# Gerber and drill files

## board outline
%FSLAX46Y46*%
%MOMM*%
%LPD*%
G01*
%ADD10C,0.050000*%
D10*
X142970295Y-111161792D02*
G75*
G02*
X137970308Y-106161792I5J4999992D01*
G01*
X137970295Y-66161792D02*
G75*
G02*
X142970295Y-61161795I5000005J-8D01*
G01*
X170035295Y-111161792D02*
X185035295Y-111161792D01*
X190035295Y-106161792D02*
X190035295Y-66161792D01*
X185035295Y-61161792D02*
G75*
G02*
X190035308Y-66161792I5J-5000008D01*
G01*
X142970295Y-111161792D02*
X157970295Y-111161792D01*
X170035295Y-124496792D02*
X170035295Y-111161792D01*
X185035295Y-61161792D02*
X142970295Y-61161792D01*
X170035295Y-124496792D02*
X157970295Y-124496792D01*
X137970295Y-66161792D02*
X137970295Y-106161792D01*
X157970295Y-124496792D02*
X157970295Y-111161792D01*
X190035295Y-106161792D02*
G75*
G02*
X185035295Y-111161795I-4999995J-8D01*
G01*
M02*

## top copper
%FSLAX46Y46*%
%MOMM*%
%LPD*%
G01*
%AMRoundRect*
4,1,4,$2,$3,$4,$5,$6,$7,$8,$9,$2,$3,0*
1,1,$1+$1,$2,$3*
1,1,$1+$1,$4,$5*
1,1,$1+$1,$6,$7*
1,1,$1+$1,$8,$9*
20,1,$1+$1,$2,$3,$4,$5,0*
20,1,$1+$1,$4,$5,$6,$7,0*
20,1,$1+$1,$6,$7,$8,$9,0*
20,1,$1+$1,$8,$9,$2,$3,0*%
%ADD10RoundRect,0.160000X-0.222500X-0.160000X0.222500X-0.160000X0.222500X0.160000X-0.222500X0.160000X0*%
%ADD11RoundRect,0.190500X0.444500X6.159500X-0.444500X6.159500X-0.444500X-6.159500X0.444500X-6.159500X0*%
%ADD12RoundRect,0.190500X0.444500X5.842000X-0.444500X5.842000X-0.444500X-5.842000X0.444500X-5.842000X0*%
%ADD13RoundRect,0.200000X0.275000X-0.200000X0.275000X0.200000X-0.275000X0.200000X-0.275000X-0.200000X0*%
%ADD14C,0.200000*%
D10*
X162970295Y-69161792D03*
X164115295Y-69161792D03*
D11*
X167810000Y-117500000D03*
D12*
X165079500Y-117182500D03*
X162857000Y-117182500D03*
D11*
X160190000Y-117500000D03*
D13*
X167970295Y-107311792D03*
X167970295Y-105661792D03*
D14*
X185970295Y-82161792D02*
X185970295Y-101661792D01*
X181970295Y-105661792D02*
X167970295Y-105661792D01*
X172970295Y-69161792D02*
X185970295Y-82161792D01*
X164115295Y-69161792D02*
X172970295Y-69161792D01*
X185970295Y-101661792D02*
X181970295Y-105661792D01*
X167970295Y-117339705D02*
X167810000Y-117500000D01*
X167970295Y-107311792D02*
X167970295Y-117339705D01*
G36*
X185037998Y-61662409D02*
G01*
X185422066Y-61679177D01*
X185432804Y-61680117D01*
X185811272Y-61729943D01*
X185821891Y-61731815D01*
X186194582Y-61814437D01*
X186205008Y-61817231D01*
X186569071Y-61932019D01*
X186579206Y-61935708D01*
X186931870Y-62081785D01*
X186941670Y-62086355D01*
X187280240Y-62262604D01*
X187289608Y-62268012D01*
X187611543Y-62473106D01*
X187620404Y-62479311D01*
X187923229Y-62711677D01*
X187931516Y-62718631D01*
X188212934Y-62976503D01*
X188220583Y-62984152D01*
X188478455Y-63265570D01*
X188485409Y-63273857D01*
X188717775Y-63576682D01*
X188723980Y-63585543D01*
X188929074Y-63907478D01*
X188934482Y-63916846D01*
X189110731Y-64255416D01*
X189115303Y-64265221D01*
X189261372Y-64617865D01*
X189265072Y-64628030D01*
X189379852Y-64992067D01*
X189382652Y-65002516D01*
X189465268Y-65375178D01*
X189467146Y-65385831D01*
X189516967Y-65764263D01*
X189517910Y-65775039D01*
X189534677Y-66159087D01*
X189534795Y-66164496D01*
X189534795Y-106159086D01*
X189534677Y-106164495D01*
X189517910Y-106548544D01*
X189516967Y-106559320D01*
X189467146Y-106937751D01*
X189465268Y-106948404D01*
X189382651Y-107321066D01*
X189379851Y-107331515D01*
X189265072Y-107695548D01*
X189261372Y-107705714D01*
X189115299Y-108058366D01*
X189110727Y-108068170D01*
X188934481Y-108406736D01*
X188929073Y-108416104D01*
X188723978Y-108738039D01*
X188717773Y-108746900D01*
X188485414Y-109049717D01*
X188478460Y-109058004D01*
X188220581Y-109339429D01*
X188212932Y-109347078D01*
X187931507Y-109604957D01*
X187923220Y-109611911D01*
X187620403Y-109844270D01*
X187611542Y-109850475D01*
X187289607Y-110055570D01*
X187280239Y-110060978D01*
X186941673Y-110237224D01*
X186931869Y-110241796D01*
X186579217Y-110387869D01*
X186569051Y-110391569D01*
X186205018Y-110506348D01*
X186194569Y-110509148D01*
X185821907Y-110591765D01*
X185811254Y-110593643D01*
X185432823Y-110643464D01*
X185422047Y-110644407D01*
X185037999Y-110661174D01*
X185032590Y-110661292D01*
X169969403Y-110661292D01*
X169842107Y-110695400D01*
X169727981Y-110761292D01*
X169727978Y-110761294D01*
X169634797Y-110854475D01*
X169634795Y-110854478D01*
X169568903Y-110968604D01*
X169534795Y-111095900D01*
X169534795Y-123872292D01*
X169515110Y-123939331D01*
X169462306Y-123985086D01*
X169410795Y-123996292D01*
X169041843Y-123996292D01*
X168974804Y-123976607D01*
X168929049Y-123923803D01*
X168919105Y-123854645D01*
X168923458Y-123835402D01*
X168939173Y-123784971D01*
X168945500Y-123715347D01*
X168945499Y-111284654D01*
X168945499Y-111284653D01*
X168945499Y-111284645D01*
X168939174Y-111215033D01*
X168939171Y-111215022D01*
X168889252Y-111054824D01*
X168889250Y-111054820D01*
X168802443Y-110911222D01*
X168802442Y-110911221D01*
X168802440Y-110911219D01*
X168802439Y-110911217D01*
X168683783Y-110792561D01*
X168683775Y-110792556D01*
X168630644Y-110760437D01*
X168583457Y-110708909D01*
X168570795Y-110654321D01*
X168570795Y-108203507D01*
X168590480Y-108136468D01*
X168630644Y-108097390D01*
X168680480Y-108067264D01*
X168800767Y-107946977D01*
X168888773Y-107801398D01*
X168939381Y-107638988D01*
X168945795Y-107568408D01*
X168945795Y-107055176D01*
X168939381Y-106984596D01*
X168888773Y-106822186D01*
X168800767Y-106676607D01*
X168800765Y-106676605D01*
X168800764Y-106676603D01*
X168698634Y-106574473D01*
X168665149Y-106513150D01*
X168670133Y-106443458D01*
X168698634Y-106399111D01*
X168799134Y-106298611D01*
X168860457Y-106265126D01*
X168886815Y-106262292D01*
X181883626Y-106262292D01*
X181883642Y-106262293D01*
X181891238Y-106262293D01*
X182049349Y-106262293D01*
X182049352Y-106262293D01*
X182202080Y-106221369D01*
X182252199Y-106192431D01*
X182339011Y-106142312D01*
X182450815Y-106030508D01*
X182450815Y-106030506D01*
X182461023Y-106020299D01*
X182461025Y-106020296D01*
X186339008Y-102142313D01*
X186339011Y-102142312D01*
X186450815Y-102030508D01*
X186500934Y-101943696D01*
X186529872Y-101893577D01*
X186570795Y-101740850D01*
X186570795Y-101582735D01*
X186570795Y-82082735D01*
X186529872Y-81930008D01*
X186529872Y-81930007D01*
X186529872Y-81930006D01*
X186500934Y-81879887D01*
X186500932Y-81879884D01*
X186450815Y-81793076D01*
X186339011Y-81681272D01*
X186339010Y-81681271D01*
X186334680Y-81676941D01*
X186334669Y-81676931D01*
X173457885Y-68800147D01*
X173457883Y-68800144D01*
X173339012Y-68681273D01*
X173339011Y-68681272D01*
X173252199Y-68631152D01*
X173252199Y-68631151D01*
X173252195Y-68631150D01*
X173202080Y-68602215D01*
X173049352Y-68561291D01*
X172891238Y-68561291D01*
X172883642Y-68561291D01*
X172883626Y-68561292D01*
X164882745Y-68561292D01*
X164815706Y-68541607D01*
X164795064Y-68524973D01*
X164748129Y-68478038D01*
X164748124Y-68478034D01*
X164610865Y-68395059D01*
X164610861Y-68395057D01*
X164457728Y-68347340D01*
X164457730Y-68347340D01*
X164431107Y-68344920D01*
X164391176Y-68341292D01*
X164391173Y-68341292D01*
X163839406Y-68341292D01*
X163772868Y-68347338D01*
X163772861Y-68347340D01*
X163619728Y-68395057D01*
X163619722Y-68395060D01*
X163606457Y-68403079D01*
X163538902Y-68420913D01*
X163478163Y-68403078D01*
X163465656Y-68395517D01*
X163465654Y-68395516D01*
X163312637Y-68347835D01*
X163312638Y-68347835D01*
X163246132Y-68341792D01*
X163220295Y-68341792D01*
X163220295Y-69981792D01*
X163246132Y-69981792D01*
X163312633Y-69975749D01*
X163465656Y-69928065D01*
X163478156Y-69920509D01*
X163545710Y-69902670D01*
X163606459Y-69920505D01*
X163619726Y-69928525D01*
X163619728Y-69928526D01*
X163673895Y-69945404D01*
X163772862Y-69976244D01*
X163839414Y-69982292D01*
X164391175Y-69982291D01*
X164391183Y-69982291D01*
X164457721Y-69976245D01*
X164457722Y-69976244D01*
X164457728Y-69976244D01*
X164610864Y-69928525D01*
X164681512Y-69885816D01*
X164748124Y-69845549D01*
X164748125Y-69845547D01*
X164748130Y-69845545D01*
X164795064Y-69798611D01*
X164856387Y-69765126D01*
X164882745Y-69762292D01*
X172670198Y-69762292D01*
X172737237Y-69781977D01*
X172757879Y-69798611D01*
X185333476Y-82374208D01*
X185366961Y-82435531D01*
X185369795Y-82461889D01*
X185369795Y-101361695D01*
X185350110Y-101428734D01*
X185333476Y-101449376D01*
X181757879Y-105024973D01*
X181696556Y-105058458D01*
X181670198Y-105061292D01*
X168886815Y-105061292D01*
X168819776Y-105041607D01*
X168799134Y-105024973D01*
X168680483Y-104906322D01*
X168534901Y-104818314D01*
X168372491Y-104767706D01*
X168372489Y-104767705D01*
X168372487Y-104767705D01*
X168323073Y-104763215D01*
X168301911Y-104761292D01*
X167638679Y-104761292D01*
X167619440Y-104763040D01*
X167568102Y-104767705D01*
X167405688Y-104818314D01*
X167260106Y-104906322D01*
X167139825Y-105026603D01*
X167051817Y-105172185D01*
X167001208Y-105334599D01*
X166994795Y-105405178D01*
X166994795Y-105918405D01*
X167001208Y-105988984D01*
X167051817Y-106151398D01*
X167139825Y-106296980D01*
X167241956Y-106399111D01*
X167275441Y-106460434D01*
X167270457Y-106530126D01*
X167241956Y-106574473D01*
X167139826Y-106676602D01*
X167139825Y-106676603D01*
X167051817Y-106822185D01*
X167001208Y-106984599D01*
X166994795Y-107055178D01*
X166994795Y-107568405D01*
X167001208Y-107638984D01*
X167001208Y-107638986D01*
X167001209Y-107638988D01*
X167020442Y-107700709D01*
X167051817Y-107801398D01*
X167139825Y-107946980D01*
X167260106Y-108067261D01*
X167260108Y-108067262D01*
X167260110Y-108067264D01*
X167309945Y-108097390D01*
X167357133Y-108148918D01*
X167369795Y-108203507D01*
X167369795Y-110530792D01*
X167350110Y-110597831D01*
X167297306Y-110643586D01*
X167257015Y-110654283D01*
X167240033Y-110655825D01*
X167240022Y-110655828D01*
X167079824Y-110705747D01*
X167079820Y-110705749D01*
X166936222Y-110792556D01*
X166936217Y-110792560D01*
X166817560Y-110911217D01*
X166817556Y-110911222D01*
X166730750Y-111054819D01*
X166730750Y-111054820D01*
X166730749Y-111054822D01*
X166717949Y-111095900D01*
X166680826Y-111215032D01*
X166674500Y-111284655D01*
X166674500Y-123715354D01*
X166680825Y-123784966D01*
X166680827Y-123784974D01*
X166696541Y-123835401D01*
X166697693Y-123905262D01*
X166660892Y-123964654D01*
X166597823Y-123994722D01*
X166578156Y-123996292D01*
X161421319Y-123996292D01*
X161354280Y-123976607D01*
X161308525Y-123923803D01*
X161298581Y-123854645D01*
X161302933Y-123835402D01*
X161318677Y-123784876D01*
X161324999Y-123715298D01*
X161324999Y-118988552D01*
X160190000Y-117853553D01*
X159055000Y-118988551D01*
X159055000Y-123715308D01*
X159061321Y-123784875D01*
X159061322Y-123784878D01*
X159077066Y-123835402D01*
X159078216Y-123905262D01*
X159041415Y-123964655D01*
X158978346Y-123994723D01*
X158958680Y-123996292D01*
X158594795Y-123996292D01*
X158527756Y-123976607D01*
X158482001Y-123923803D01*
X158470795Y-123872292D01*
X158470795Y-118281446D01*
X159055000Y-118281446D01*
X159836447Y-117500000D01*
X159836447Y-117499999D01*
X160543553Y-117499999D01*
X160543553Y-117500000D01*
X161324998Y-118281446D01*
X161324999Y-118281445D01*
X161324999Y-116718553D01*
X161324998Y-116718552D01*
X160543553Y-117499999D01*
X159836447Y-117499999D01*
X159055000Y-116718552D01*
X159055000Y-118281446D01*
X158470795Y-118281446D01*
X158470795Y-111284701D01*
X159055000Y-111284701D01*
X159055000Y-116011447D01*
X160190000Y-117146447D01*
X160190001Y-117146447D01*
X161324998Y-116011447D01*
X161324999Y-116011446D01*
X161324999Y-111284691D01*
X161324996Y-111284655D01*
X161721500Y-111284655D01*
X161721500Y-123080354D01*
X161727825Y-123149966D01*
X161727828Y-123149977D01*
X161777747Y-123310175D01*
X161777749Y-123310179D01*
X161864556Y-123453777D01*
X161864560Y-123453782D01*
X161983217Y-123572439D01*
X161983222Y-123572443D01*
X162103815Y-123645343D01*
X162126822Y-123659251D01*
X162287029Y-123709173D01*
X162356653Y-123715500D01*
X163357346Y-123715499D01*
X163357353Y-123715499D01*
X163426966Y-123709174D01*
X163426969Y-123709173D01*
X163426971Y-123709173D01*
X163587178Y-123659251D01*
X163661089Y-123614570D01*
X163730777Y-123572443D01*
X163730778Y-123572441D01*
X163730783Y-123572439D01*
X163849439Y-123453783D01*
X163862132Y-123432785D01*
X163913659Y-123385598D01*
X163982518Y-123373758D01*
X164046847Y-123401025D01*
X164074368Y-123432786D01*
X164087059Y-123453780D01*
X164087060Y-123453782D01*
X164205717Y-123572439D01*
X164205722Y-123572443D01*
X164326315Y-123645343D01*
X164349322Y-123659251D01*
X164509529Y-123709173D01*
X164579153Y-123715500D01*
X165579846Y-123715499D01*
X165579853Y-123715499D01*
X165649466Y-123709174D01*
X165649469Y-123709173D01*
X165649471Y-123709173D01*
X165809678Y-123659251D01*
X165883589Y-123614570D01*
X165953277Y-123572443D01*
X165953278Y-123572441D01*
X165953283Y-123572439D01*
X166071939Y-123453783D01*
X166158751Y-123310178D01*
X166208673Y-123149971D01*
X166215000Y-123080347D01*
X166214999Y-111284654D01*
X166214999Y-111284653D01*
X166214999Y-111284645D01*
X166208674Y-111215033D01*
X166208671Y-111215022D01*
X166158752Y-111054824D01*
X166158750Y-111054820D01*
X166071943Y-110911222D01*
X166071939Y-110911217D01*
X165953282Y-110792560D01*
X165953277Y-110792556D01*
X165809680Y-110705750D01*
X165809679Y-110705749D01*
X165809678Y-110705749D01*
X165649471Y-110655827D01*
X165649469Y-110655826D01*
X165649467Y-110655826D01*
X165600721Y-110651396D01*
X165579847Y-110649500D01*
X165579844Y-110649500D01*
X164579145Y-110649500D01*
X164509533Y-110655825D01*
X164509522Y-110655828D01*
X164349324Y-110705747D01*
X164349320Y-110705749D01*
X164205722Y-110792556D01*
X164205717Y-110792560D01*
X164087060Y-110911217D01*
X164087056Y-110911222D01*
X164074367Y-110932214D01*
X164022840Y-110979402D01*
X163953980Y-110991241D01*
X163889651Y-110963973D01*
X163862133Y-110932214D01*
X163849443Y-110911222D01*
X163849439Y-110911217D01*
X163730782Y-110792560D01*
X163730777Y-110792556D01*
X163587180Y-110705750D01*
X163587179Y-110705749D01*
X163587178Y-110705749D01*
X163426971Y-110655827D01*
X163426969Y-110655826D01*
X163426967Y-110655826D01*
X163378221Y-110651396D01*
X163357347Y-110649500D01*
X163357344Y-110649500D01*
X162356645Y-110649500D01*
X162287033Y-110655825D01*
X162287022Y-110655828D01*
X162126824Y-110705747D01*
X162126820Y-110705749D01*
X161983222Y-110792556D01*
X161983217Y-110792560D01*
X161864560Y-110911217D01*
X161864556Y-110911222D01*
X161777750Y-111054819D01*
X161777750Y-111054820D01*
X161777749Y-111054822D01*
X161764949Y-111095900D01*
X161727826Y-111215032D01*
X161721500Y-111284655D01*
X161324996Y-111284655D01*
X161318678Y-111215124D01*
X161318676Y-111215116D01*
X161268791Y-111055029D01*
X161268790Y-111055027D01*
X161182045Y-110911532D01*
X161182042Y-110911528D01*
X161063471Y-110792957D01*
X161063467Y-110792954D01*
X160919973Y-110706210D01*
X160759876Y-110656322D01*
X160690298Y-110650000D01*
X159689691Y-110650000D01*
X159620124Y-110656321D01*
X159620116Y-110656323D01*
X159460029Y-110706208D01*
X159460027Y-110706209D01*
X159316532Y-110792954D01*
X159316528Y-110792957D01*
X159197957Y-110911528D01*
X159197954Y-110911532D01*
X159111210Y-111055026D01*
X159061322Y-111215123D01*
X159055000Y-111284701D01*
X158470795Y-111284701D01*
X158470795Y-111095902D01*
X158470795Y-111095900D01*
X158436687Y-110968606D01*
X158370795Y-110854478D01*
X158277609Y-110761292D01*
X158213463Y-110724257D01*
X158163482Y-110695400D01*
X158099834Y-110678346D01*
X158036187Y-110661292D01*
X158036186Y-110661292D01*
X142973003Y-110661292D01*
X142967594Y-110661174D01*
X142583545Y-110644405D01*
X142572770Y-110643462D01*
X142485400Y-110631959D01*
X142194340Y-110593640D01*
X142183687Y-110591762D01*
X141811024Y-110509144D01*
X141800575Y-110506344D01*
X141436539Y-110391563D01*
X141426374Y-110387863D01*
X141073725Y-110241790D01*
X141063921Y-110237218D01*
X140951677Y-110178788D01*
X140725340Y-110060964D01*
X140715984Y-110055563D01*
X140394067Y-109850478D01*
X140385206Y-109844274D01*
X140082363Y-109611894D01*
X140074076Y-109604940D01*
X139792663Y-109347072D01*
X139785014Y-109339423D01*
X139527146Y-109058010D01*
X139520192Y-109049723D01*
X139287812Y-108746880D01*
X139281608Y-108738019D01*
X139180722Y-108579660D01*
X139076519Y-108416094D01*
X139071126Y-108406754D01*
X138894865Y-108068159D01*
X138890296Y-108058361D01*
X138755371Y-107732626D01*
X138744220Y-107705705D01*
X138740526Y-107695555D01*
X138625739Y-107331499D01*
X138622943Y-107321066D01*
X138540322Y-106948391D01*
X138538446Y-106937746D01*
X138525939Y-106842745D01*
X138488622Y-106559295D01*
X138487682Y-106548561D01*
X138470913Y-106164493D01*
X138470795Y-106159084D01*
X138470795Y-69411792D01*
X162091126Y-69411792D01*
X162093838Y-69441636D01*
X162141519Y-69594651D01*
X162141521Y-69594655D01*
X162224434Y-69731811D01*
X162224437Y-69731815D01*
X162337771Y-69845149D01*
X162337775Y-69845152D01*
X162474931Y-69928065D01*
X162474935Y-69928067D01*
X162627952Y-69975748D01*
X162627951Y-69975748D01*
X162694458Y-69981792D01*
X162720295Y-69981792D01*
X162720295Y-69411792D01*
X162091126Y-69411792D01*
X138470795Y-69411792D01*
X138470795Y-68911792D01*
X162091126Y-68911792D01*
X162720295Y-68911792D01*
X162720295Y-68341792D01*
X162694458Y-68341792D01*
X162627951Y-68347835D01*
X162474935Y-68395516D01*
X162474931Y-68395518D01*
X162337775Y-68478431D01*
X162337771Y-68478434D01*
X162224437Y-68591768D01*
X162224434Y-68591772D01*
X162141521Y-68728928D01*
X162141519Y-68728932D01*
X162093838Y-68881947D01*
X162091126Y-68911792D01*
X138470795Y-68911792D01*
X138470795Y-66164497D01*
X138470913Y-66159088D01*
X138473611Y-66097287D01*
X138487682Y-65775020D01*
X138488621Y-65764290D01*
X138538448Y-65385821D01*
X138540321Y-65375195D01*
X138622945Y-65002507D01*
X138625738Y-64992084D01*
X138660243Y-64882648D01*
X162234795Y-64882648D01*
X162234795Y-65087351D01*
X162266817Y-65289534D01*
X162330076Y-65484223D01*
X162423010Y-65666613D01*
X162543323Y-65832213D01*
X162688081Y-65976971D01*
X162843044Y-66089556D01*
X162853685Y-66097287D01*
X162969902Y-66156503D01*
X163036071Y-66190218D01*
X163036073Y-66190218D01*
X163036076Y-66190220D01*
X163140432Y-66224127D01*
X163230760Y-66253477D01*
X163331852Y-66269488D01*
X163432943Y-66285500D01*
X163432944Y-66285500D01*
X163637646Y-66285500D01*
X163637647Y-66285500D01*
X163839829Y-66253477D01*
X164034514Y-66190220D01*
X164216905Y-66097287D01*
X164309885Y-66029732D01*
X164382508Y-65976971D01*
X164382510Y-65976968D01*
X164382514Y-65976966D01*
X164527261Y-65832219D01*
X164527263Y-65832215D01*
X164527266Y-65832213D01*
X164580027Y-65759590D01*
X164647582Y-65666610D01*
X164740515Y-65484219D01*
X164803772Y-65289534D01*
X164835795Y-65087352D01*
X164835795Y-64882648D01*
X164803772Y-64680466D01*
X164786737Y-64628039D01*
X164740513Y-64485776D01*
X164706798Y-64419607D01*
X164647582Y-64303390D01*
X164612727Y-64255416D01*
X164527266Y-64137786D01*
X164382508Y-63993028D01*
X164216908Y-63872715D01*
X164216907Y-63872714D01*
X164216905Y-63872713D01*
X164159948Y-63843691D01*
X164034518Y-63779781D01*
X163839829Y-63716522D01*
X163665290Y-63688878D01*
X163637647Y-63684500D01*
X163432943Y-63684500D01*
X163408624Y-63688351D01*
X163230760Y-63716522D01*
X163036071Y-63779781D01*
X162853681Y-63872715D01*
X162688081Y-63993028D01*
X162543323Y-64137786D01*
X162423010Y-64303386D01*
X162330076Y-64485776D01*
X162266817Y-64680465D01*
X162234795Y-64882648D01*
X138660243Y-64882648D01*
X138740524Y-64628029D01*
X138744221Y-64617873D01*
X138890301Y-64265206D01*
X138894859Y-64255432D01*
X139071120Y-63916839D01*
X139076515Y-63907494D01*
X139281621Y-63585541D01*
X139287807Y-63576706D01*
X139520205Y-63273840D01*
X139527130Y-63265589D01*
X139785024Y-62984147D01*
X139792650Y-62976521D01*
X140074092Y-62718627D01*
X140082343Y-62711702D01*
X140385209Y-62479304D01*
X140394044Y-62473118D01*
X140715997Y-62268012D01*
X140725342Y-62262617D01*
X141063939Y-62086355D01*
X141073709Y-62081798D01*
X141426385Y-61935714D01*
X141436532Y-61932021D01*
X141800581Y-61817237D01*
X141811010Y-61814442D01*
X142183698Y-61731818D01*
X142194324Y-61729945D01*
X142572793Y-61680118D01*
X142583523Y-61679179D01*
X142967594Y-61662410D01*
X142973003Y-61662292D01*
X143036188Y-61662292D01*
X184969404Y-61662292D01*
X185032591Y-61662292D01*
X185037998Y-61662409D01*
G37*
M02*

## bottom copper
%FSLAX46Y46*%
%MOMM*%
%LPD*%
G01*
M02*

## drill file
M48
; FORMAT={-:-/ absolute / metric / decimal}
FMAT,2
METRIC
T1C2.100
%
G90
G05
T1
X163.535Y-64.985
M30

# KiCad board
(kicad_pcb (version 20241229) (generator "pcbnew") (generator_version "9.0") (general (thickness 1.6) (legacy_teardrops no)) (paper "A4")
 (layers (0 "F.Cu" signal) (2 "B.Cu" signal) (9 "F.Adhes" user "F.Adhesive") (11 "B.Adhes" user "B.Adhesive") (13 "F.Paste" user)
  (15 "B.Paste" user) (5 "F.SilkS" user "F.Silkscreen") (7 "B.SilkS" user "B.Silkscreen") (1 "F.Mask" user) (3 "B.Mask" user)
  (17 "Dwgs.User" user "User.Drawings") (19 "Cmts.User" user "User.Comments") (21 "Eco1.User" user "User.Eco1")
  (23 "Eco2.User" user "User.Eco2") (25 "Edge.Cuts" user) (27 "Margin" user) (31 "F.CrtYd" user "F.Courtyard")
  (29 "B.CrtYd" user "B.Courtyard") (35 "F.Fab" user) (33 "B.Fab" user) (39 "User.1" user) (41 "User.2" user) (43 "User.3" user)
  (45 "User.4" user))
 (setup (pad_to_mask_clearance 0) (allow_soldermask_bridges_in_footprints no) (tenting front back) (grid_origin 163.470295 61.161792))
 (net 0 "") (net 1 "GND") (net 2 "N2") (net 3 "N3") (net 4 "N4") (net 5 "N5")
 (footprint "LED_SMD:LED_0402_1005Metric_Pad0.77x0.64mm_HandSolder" (layer "F.Cu") (at 163.542795 69.161792)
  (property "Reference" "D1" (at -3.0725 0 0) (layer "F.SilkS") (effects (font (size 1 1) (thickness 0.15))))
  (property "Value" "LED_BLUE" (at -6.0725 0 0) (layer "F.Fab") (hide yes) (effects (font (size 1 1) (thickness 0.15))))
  (pad "1" smd roundrect (at -0.5725 0) (size 0.765 0.64) (layers "F.Cu" "F.Mask" "F.Paste") (roundrect_rratio 0.25) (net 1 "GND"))
  (pad "2" smd roundrect (at 0.5725 0) (size 0.765 0.64) (layers "F.Cu" "F.Mask" "F.Paste") (roundrect_rratio 0.25) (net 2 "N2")))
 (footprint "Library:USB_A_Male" (layer "F.Cu") (at 164 117.1825 180)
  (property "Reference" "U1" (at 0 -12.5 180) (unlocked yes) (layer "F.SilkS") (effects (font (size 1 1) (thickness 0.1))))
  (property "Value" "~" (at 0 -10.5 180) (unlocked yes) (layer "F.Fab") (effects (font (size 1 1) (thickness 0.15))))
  (pad "1" smd roundrect (at -3.81 -0.3175 180) (size 1.27 12.7) (layers "F.Cu" "F.Mask" "F.Paste") (roundrect_rratio 0.15) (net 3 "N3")
   (thermal_bridge_angle 45))
  (pad "2" smd roundrect (at -1.0795 0 180) (size 1.27 12.065) (layers "F.Cu" "F.Mask" "F.Paste") (roundrect_rratio 0.15) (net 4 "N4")
   (thermal_bridge_angle 45))
  (pad "3" smd roundrect (at 1.143 0 180) (size 1.27 12.065) (layers "F.Cu" "F.Mask" "F.Paste") (roundrect_rratio 0.15) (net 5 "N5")
   (thermal_bridge_angle 45))
  (pad "4" smd roundrect (at 3.81 -0.3175 180) (size 1.27 12.7) (layers "F.Cu" "F.Mask" "F.Paste") (roundrect_rratio 0.15) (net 1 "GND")
   (thermal_bridge_angle 45)))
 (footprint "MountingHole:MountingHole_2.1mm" (layer "F.Cu") (at 163.535295 64.985 180)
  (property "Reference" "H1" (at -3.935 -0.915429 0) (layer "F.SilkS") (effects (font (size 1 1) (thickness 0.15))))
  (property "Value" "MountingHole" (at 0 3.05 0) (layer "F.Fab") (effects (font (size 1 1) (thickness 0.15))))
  (pad "" np_thru_hole circle (at 0 0 180) (size 2.1 2.1) (drill 2.1) (layers "*.Cu" "*.Mask")))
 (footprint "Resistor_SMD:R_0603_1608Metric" (layer "F.Cu") (at 167.970295 106.486792 90)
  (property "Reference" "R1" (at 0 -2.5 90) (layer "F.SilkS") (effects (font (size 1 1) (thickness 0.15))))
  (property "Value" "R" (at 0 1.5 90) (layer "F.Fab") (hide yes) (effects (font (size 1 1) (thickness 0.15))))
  (pad "1" smd roundrect (at -0.825 0 90) (size 0.8 0.95) (layers "F.Cu" "F.Mask" "F.Paste") (roundrect_rratio 0.25) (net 3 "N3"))
  (pad "2" smd roundrect (at 0.825 0 90) (size 0.8 0.95) (layers "F.Cu" "F.Mask" "F.Paste") (roundrect_rratio 0.25) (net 2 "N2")))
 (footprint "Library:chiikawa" (layer "F.Cu") (at 161.970295 86.661792)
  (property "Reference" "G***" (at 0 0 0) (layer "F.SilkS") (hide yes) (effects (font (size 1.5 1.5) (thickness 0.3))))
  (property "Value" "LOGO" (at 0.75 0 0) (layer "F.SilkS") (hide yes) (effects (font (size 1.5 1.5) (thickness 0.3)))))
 (gr_arc (start 142.970295 111.161792) (mid 139.434767 109.697324) (end 137.970295 106.161792) (stroke (width 0.05) (type default))
  (layer "Edge.Cuts"))
 (gr_arc (start 137.970295 66.161792) (mid 139.434764 62.626261) (end 142.970295 61.161792) (stroke (width 0.05) (type default))
  (layer "Edge.Cuts"))
 (gr_line (start 170.035295 111.161792) (end 185.035295 111.161792) (stroke (width 0.05) (type solid)) (layer "Edge.Cuts"))
 (gr_line (start 190.035295 106.161792) (end 190.035295 66.161792) (stroke (width 0.05) (type solid)) (layer "Edge.Cuts"))
 (gr_arc (start 185.035295 61.161792) (mid 188.570835 62.626256) (end 190.035295 66.161792) (stroke (width 0.05) (type default))
  (layer "Edge.Cuts"))
 (gr_line (start 142.970295 111.161792) (end 157.970295 111.161792) (stroke (width 0.05) (type solid)) (layer "Edge.Cuts"))
 (gr_line (start 170.035295 124.496792) (end 170.035295 111.161792) (stroke (width 0.05) (type solid)) (layer "Edge.Cuts"))
 (gr_line (start 185.035295 61.161792) (end 142.970295 61.161792) (stroke (width 0.05) (type solid)) (layer "Edge.Cuts"))
 (gr_line (start 170.035295 124.496792) (end 157.970295 124.496792) (stroke (width 0.05) (type solid)) (layer "Edge.Cuts"))
 (gr_line (start 137.970295 66.161792) (end 137.970295 106.161792) (stroke (width 0.05) (type solid)) (layer "Edge.Cuts"))
 (gr_line (start 157.970295 124.496792) (end 157.970295 111.161792) (stroke (width 0.05) (type solid)) (layer "Edge.Cuts"))
 (gr_arc (start 190.035295 106.161792) (mid 188.570831 109.697329) (end 185.035295 111.161792) (stroke (width 0.05) (type default))
  (layer "Edge.Cuts"))
 (segment (start 185.970295 82.161792) (end 185.970295 101.661792) (width 0.2) (layer "F.Cu") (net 2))
 (segment (start 181.970295 105.661792) (end 167.970295 105.661792) (width 0.2) (layer "F.Cu") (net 2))
 (segment (start 172.970295 69.161792) (end 185.970295 82.161792) (width 0.2) (layer "F.Cu") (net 2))
 (segment (start 164.115295 69.161792) (end 172.970295 69.161792) (width 0.2) (layer "F.Cu") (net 2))
 (segment (start 185.970295 101.661792) (end 181.970295 105.661792) (width 0.2) (layer "F.Cu") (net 2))
 (segment (start 167.970295 117.339705) (end 167.81 117.5) (width 0.2) (layer "F.Cu") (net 3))
 (segment (start 167.970295 107.311792) (end 167.970295 117.339705) (width 0.2) (layer "F.Cu") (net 3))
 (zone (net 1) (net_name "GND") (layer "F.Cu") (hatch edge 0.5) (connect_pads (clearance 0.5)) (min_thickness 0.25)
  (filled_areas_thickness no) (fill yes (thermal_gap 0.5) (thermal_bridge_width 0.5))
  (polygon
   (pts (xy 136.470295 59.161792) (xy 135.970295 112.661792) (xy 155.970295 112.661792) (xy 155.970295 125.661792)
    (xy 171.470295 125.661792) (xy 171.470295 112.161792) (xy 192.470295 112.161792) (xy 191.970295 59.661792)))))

